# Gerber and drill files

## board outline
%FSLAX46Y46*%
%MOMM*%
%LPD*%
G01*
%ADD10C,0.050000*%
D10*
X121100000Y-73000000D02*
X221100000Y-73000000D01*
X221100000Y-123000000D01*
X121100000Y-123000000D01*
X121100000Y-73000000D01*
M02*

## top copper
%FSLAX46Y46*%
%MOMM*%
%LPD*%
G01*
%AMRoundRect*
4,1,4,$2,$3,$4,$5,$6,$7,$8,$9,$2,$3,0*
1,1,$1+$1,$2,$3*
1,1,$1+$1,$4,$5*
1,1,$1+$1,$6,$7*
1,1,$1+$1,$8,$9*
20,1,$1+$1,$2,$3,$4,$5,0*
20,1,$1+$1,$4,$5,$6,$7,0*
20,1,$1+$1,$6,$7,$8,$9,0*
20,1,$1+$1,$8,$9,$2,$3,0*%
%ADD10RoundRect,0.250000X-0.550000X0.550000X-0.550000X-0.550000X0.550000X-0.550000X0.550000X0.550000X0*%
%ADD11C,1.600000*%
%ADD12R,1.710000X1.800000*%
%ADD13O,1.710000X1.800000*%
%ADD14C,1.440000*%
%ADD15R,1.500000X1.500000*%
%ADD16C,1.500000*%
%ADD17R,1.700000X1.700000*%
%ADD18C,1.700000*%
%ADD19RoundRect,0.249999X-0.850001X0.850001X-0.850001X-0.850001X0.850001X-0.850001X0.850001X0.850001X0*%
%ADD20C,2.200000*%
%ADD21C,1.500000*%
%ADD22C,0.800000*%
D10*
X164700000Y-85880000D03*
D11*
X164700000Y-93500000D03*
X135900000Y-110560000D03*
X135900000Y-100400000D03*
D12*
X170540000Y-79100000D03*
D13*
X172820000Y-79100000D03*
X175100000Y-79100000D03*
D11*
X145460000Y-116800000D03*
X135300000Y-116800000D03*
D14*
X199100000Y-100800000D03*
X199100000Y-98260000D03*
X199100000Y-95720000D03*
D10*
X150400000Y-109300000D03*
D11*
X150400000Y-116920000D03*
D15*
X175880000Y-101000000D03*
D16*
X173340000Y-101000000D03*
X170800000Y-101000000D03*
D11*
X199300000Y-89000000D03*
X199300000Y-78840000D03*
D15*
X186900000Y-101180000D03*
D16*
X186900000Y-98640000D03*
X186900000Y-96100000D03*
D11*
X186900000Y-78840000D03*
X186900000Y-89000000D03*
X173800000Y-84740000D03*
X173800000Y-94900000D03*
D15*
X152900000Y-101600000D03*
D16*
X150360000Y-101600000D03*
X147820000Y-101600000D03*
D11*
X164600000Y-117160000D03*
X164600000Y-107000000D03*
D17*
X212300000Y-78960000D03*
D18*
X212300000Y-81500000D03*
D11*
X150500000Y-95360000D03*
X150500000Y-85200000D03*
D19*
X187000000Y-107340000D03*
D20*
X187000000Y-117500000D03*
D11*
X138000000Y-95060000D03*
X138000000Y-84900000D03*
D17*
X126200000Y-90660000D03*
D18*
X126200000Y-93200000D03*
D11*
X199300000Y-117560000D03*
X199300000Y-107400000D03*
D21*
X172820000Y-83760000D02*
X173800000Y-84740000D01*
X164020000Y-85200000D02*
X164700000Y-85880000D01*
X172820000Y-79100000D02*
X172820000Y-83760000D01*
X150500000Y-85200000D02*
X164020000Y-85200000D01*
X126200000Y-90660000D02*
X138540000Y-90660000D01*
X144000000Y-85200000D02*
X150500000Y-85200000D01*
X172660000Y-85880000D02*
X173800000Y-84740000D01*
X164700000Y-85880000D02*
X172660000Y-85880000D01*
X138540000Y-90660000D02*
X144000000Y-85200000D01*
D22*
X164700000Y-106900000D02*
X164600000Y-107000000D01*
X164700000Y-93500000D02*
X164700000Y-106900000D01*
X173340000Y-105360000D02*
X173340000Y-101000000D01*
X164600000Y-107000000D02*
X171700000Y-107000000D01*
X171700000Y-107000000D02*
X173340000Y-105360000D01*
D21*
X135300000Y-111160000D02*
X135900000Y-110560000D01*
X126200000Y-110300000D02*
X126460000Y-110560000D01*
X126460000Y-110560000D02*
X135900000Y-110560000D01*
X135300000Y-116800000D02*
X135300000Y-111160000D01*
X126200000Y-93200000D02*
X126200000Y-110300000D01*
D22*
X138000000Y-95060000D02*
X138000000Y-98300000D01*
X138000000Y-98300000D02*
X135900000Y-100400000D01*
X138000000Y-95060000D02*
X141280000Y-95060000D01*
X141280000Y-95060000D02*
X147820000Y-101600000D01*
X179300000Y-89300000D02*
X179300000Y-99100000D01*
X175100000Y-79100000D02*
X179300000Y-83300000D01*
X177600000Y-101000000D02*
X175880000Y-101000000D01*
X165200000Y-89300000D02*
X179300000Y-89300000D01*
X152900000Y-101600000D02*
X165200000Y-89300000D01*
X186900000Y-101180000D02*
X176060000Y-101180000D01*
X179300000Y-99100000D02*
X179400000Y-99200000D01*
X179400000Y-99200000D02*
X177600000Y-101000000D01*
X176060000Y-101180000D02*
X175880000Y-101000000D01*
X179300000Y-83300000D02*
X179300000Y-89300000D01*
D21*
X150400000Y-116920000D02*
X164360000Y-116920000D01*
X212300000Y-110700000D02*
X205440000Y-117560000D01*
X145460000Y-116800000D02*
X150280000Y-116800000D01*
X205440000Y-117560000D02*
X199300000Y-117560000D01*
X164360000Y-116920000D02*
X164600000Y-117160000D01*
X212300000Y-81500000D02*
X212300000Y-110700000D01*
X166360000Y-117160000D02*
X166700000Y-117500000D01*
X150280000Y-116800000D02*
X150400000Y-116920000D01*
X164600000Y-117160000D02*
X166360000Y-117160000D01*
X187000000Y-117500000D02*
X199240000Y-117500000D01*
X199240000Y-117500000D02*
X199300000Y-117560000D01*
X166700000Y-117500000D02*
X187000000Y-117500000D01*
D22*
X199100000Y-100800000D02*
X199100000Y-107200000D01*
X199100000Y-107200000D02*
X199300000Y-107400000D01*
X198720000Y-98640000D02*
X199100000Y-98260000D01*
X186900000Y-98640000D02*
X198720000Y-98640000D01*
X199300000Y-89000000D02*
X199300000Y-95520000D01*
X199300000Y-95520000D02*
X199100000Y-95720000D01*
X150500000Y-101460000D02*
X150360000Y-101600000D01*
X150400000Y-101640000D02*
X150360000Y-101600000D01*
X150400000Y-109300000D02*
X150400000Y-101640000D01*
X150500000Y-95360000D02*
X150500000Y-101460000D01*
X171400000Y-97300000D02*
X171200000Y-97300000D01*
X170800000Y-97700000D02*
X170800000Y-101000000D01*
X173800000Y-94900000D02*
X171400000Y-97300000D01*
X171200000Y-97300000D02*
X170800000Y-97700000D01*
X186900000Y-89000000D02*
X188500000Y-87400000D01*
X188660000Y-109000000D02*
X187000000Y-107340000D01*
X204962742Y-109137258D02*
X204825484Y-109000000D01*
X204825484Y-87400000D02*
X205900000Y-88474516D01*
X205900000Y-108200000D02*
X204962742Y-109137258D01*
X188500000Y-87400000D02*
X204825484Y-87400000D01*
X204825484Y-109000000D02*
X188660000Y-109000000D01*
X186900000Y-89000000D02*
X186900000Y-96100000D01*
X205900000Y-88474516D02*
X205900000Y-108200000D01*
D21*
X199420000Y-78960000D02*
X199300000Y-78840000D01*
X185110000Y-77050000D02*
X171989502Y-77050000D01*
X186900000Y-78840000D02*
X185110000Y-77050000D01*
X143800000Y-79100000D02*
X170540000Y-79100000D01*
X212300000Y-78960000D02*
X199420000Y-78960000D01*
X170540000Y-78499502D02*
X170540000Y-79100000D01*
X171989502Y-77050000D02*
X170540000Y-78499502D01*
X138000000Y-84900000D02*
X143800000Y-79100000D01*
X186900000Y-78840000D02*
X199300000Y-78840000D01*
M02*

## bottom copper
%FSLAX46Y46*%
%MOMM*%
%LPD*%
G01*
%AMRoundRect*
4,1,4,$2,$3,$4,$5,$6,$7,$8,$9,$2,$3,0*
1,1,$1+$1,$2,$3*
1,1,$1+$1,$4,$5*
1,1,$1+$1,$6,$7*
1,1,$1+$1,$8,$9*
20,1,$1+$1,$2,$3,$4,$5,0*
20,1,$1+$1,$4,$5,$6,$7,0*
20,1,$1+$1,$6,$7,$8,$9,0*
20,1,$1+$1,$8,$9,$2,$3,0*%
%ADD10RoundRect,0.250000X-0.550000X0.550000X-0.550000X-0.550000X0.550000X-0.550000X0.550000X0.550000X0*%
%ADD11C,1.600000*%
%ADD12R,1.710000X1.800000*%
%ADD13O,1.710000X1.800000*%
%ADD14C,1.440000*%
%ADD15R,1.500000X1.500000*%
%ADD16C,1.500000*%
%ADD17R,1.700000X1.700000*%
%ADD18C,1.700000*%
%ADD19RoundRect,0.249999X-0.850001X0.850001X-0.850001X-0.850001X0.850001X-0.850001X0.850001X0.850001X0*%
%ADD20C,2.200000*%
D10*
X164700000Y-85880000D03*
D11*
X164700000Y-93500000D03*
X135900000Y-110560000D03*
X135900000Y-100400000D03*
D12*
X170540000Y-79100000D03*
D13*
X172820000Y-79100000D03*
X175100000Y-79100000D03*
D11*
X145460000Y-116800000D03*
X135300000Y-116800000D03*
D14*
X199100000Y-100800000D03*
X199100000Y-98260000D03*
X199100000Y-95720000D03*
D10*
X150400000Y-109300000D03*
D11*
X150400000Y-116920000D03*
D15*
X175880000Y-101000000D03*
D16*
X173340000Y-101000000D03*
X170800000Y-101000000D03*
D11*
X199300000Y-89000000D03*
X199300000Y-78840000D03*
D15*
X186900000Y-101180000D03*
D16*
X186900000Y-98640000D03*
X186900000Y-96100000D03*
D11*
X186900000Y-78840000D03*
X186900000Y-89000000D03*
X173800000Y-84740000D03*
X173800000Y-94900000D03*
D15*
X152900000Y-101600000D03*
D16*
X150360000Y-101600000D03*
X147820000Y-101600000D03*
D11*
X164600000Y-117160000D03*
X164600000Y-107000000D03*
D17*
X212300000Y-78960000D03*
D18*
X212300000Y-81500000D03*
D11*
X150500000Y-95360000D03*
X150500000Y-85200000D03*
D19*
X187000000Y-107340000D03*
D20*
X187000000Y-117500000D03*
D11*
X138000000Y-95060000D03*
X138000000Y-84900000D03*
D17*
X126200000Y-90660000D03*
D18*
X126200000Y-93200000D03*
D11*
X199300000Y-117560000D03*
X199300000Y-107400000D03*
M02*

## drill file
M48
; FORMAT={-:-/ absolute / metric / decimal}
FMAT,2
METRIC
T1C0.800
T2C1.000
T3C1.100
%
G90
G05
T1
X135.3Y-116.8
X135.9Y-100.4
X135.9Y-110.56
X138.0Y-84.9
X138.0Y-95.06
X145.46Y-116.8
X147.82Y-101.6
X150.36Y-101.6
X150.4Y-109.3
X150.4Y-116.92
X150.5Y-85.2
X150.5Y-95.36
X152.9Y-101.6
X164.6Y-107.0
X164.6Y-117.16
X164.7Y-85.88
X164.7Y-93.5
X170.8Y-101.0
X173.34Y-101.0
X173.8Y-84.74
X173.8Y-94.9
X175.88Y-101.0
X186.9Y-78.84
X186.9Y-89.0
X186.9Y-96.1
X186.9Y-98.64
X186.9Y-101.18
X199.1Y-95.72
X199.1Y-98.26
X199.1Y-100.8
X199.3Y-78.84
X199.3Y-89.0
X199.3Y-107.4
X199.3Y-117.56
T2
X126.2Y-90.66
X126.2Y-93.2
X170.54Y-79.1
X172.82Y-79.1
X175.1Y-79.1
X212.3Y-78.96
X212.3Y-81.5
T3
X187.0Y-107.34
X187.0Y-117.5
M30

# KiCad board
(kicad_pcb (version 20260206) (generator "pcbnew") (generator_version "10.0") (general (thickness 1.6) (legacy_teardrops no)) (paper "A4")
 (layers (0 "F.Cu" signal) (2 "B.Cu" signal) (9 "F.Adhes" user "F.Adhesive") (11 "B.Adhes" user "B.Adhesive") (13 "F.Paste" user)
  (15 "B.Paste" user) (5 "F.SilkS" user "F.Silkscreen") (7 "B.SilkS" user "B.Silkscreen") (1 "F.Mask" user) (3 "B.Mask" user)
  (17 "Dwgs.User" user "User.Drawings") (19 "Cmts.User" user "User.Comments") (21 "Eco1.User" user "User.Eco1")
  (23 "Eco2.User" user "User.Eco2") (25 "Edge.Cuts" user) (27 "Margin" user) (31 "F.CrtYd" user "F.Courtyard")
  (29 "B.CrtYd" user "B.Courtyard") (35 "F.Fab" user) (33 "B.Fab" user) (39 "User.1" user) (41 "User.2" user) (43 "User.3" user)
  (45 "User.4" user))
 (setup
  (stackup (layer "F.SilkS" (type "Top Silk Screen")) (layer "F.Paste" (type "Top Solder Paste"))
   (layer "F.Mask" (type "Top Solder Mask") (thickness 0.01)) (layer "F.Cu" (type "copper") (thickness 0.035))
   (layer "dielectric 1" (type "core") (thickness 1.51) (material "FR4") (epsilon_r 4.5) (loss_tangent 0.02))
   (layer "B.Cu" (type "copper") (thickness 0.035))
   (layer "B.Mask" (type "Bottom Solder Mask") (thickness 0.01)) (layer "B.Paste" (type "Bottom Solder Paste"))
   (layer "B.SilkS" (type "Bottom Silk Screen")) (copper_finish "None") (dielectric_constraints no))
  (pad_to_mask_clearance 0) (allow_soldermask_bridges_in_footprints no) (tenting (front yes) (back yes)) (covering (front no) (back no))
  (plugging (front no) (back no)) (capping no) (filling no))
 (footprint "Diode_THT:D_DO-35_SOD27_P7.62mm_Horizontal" (layer "F.Cu") (at 164.7 85.88 -90)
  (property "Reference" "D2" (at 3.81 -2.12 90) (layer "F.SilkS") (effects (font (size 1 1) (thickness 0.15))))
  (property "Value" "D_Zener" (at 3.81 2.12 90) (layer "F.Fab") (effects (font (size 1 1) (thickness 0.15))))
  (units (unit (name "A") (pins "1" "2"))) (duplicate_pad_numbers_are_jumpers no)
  (pad "1" thru_hole roundrect (at 0 0 270) (size 1.6 1.6) (drill 0.8) (layers "*.Cu" "*.Mask") (remove_unused_layers no)
   (roundrect_rratio 0.15625) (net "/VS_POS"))
  (pad "2" thru_hole circle (at 7.62 0 270) (size 1.6 1.6) (drill 0.8) (layers "*.Cu" "*.Mask") (remove_unused_layers no) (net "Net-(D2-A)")))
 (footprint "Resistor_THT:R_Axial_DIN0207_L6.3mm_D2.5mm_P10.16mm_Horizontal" (layer "F.Cu") (at 135.9 110.56 90)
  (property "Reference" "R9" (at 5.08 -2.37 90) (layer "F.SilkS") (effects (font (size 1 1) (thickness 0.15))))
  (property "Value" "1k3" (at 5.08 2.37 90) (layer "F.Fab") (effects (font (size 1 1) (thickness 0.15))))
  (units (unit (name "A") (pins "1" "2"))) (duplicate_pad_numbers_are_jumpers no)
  (pad "1" thru_hole circle (at 0 0 90) (size 1.6 1.6) (drill 0.8) (layers "*.Cu" "*.Mask") (remove_unused_layers no) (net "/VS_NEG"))
  (pad "2" thru_hole circle (at 10.16 0 90) (size 1.6 1.6) (drill 0.8) (layers "*.Cu" "*.Mask") (remove_unused_layers no) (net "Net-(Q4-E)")))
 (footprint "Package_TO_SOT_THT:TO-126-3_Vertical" (layer "F.Cu") (at 170.54 79.1)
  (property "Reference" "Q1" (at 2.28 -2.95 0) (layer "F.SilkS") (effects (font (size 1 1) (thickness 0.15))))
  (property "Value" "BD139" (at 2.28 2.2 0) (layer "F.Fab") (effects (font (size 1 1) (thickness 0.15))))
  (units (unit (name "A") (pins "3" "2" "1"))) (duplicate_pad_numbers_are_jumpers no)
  (pad "1" thru_hole rect (at 0 0) (size 1.71 1.8) (drill 1) (layers "*.Cu" "*.Mask") (remove_unused_layers no) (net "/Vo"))
  (pad "2" thru_hole oval (at 2.28 0) (size 1.71 1.8) (drill 1) (layers "*.Cu" "*.Mask") (remove_unused_layers no) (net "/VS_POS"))
  (pad "3" thru_hole oval (at 4.56 0) (size 1.71 1.8) (drill 1) (layers "*.Cu" "*.Mask") (remove_unused_layers no) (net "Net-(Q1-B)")))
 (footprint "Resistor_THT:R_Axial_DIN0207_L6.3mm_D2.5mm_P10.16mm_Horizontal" (layer "F.Cu") (at 145.46 116.8 180)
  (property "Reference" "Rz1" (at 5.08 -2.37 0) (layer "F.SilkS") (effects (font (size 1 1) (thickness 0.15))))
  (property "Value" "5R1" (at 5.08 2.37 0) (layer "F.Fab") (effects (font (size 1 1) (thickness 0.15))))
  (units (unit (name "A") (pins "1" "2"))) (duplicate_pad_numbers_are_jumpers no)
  (pad "1" thru_hole circle (at 0 0 180) (size 1.6 1.6) (drill 0.8) (layers "*.Cu" "*.Mask") (remove_unused_layers no) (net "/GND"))
  (pad "2" thru_hole circle (at 10.16 0 180) (size 1.6 1.6) (drill 0.8) (layers "*.Cu" "*.Mask") (remove_unused_layers no) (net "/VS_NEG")))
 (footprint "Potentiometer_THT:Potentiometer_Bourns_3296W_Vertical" (layer "F.Cu") (at 199.1 100.8 -90)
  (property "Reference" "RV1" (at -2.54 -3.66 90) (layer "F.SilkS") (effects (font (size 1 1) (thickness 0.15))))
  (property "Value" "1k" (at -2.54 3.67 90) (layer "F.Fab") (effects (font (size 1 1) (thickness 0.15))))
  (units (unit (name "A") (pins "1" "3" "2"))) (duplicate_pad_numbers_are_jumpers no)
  (pad "1" thru_hole circle (at 0 0 270) (size 1.44 1.44) (drill 0.8) (layers "*.Cu" "*.Mask") (remove_unused_layers no)
   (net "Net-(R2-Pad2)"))
  (pad "2" thru_hole circle (at -2.54 0 270) (size 1.44 1.44) (drill 0.8) (layers "*.Cu" "*.Mask") (remove_unused_layers no)
   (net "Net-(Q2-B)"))
  (pad "3" thru_hole circle (at -5.08 0 270) (size 1.44 1.44) (drill 0.8) (layers "*.Cu" "*.Mask") (remove_unused_layers no)
   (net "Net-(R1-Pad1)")))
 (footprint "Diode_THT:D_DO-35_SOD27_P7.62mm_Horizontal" (layer "F.Cu") (at 150.4 109.3 -90)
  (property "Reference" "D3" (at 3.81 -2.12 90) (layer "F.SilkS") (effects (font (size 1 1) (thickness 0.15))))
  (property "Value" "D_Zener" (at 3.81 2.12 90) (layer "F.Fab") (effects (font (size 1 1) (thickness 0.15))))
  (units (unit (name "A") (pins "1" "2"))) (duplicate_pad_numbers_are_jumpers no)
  (pad "1" thru_hole roundrect (at 0 0 270) (size 1.6 1.6) (drill 0.8) (layers "*.Cu" "*.Mask") (remove_unused_layers no)
   (roundrect_rratio 0.15625) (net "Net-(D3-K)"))
  (pad "2" thru_hole circle (at 7.62 0 270) (size 1.6 1.6) (drill 0.8) (layers "*.Cu" "*.Mask") (remove_unused_layers no) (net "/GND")))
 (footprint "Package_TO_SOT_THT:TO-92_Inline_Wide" (layer "F.Cu") (at 175.88 101 180)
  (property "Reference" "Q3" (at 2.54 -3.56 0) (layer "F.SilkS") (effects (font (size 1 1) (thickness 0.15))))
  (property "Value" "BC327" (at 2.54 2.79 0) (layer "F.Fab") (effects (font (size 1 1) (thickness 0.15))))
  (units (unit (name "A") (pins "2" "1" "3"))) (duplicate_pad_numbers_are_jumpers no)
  (pad "1" thru_hole rect (at 0 0 180) (size 1.5 1.5) (drill 0.8) (layers "*.Cu" "*.Mask") (remove_unused_layers no) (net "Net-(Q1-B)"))
  (pad "2" thru_hole circle (at 2.54 0 180) (size 1.5 1.5) (drill 0.8) (layers "*.Cu" "*.Mask") (remove_unused_layers no) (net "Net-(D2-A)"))
  (pad "3" thru_hole circle (at 5.08 0 180) (size 1.5 1.5) (drill 0.8) (layers "*.Cu" "*.Mask") (remove_unused_layers no) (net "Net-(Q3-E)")))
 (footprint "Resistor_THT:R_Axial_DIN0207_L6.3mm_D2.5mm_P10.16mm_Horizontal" (layer "F.Cu") (at 199.3 89 90)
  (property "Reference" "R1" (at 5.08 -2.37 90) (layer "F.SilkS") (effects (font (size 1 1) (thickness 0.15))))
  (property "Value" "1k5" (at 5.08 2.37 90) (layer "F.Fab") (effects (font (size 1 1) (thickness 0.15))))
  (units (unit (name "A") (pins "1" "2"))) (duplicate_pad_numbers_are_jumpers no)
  (pad "1" thru_hole circle (at 0 0 90) (size 1.6 1.6) (drill 0.8) (layers "*.Cu" "*.Mask") (remove_unused_layers no) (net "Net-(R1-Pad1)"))
  (pad "2" thru_hole circle (at 10.16 0 90) (size 1.6 1.6) (drill 0.8) (layers "*.Cu" "*.Mask") (remove_unused_layers no) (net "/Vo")))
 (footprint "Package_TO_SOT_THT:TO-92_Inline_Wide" (layer "F.Cu") (at 186.9 101.18 90)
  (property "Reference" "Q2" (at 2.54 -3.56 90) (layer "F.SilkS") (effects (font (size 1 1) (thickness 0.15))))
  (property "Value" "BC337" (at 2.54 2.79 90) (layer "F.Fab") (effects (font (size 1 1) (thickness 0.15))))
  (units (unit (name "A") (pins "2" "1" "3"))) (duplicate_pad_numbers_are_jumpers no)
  (pad "1" thru_hole rect (at 0 0 90) (size 1.5 1.5) (drill 0.8) (layers "*.Cu" "*.Mask") (remove_unused_layers no) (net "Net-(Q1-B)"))
  (pad "2" thru_hole circle (at 2.54 0 90) (size 1.5 1.5) (drill 0.8) (layers "*.Cu" "*.Mask") (remove_unused_layers no) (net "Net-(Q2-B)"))
  (pad "3" thru_hole circle (at 5.08 0 90) (size 1.5 1.5) (drill 0.8) (layers "*.Cu" "*.Mask") (remove_unused_layers no) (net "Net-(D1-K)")))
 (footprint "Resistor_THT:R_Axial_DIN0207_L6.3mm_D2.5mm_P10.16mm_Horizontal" (layer "F.Cu") (at 186.9 78.84 -90)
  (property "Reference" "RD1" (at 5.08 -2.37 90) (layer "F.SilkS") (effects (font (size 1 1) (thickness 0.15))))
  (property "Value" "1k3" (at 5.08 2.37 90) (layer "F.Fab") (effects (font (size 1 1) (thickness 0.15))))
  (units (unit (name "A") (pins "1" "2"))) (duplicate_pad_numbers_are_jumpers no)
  (pad "1" thru_hole circle (at 0 0 270) (size 1.6 1.6) (drill 0.8) (layers "*.Cu" "*.Mask") (remove_unused_layers no) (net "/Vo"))
  (pad "2" thru_hole circle (at 10.16 0 270) (size 1.6 1.6) (drill 0.8) (layers "*.Cu" "*.Mask") (remove_unused_layers no)
   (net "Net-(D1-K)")))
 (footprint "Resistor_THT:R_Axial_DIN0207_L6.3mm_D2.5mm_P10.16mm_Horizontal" (layer "F.Cu") (at 173.8 84.74 -90)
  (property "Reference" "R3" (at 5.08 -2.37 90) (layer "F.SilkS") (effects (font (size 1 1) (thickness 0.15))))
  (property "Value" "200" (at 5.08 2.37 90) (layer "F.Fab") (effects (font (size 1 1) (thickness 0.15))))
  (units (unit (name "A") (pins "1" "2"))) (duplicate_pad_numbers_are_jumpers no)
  (pad "1" thru_hole circle (at 0 0 270) (size 1.6 1.6) (drill 0.8) (layers "*.Cu" "*.Mask") (remove_unused_layers no) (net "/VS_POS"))
  (pad "2" thru_hole circle (at 10.16 0 270) (size 1.6 1.6) (drill 0.8) (layers "*.Cu" "*.Mask") (remove_unused_layers no)
   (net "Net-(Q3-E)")))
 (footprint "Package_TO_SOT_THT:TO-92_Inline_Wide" (layer "F.Cu") (at 152.9 101.6 180)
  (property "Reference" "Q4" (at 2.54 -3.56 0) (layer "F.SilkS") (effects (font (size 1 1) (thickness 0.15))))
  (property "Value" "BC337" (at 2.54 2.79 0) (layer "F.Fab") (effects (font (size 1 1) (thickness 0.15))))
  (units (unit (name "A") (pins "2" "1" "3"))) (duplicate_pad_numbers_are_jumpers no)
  (pad "1" thru_hole rect (at 0 0 180) (size 1.5 1.5) (drill 0.8) (layers "*.Cu" "*.Mask") (remove_unused_layers no) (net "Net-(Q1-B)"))
  (pad "2" thru_hole circle (at 2.54 0 180) (size 1.5 1.5) (drill 0.8) (layers "*.Cu" "*.Mask") (remove_unused_layers no) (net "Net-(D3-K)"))
  (pad "3" thru_hole circle (at 5.08 0 180) (size 1.5 1.5) (drill 0.8) (layers "*.Cu" "*.Mask") (remove_unused_layers no) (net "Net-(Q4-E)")))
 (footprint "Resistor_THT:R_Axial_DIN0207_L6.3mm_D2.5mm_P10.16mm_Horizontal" (layer "F.Cu") (at 164.6 117.16 90)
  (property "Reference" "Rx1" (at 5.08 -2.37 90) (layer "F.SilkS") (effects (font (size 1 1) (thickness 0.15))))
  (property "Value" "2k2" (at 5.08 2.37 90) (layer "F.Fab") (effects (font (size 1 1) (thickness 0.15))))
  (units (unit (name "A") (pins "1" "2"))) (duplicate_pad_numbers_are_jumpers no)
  (pad "1" thru_hole circle (at 0 0 90) (size 1.6 1.6) (drill 0.8) (layers "*.Cu" "*.Mask") (remove_unused_layers no) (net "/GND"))
  (pad "2" thru_hole circle (at 10.16 0 90) (size 1.6 1.6) (drill 0.8) (layers "*.Cu" "*.Mask") (remove_unused_layers no) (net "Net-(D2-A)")))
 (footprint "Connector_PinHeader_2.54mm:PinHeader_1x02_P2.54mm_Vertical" (layer "F.Cu") (at 212.3 78.96)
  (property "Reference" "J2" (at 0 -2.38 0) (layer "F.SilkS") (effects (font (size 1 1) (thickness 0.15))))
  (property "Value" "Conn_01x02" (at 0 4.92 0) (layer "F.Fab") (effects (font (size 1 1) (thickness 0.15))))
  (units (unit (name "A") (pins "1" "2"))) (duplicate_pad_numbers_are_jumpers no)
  (pad "1" thru_hole rect (at 0 0) (size 1.7 1.7) (drill 1) (layers "*.Cu" "*.Mask") (remove_unused_layers no) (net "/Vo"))
  (pad "2" thru_hole circle (at 0 2.54) (size 1.7 1.7) (drill 1) (layers "*.Cu" "*.Mask") (remove_unused_layers no) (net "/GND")))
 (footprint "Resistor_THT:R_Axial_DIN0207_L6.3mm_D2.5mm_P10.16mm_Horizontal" (layer "F.Cu") (at 150.5 95.36 90)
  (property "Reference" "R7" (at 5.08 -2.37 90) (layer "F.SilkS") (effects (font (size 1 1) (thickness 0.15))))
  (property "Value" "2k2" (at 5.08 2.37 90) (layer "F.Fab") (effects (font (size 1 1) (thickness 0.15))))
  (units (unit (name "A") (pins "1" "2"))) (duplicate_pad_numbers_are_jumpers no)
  (pad "1" thru_hole circle (at 0 0 90) (size 1.6 1.6) (drill 0.8) (layers "*.Cu" "*.Mask") (remove_unused_layers no) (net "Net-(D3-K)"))
  (pad "2" thru_hole circle (at 10.16 0 90) (size 1.6 1.6) (drill 0.8) (layers "*.Cu" "*.Mask") (remove_unused_layers no) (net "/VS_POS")))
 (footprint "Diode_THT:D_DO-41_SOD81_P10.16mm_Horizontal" (layer "F.Cu") (at 187 107.34 -90)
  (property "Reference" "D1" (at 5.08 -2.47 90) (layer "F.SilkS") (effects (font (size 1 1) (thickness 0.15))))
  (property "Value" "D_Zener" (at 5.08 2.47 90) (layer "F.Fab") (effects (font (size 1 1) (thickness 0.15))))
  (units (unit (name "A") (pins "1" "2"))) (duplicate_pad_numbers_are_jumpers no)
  (pad "1" thru_hole roundrect (at 0 0 270) (size 2.2 2.2) (drill 1.1) (layers "*.Cu" "*.Mask") (remove_unused_layers no)
   (roundrect_rratio 0.113636) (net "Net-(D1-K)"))
  (pad "2" thru_hole circle (at 10.16 0 270) (size 2.2 2.2) (drill 1.1) (layers "*.Cu" "*.Mask") (remove_unused_layers no) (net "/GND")))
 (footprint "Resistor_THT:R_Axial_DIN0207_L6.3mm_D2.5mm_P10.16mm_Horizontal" (layer "F.Cu") (at 138 95.06 90)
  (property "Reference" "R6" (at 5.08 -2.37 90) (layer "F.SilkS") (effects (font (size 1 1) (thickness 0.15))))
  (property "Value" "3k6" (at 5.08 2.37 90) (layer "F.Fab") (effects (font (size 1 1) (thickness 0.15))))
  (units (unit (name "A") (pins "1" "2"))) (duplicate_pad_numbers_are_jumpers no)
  (pad "1" thru_hole circle (at 0 0 90) (size 1.6 1.6) (drill 0.8) (layers "*.Cu" "*.Mask") (remove_unused_layers no) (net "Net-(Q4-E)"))
  (pad "2" thru_hole circle (at 10.16 0 90) (size 1.6 1.6) (drill 0.8) (layers "*.Cu" "*.Mask") (remove_unused_layers no) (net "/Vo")))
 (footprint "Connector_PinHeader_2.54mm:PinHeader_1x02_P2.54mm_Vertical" (layer "F.Cu") (at 126.2 90.66)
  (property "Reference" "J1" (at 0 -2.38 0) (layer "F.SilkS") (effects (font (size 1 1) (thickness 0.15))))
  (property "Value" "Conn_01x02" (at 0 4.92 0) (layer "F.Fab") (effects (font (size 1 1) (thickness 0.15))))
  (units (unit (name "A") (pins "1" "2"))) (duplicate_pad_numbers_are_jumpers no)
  (pad "1" thru_hole rect (at 0 0) (size 1.7 1.7) (drill 1) (layers "*.Cu" "*.Mask") (remove_unused_layers no) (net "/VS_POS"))
  (pad "2" thru_hole circle (at 0 2.54) (size 1.7 1.7) (drill 1) (layers "*.Cu" "*.Mask") (remove_unused_layers no) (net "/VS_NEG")))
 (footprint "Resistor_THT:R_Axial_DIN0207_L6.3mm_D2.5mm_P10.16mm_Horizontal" (layer "F.Cu") (at 199.3 117.56 90)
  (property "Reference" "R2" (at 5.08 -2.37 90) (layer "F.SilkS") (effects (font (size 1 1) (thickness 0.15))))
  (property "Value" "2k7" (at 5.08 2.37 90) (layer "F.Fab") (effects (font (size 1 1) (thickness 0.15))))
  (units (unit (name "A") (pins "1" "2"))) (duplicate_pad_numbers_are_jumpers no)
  (pad "1" thru_hole circle (at 0 0 90) (size 1.6 1.6) (drill 0.8) (layers "*.Cu" "*.Mask") (remove_unused_layers no) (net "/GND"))
  (pad "2" thru_hole circle (at 10.16 0 90) (size 1.6 1.6) (drill 0.8) (layers "*.Cu" "*.Mask") (remove_unused_layers no)
   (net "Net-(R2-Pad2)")))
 (gr_rect (start 121.1 73) (end 221.1 123) (stroke (width 0.05) (type default)) (fill no) (layer "Edge.Cuts"))
 (segment (start 172.82 83.76) (end 173.8 84.74) (width 1.5) (layer "F.Cu") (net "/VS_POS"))
 (segment (start 164.02 85.2) (end 164.7 85.88) (width 1.5) (layer "F.Cu") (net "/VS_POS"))
 (segment (start 172.82 79.1) (end 172.82 83.76) (width 1.5) (layer "F.Cu") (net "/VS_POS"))
 (segment (start 150.5 85.2) (end 164.02 85.2) (width 1.5) (layer "F.Cu") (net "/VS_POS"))
 (segment (start 126.2 90.66) (end 138.54 90.66) (width 1.5) (layer "F.Cu") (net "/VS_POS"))
 (segment (start 144 85.2) (end 150.5 85.2) (width 1.5) (layer "F.Cu") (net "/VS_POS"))
 (segment (start 172.66 85.88) (end 173.8 84.74) (width 1.5) (layer "F.Cu") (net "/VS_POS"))
 (segment (start 164.7 85.88) (end 172.66 85.88) (width 1.5) (layer "F.Cu") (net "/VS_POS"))
 (segment (start 138.54 90.66) (end 144 85.2) (width 1.5) (layer "F.Cu") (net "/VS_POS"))
 (segment (start 164.7 106.9) (end 164.6 107) (width 0.8) (layer "F.Cu") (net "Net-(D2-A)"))
 (segment (start 164.7 93.5) (end 164.7 106.9) (width 0.8) (layer "F.Cu") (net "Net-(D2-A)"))
 (segment (start 173.34 105.36) (end 173.34 101) (width 0.8) (layer "F.Cu") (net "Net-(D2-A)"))
 (segment (start 164.6 107) (end 171.7 107) (width 0.8) (layer "F.Cu") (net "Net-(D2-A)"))
 (segment (start 171.7 107) (end 173.34 105.36) (width 0.8) (layer "F.Cu") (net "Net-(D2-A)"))
 (segment (start 135.3 111.16) (end 135.9 110.56) (width 1.5) (layer "F.Cu") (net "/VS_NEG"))
 (segment (start 126.2 110.3) (end 126.46 110.56) (width 1.5) (layer "F.Cu") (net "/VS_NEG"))
 (segment (start 126.46 110.56) (end 135.9 110.56) (width 1.5) (layer "F.Cu") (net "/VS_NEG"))
 (segment (start 135.3 116.8) (end 135.3 111.16) (width 1.5) (layer "F.Cu") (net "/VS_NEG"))
 (segment (start 126.2 93.2) (end 126.2 110.3) (width 1.5) (layer "F.Cu") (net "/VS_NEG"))
 (segment (start 138 95.06) (end 138 98.3) (width 0.8) (layer "F.Cu") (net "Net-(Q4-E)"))
 (segment (start 138 98.3) (end 135.9 100.4) (width 0.8) (layer "F.Cu") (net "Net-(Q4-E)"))
 (segment (start 138 95.06) (end 141.28 95.06) (width 0.8) (layer "F.Cu") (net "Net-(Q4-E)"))
 (segment (start 141.28 95.06) (end 147.82 101.6) (width 0.8) (layer "F.Cu") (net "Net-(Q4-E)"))
 (segment (start 179.3 89.3) (end 179.3 99.1) (width 0.8) (layer "F.Cu") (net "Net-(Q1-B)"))
 (segment (start 175.1 79.1) (end 179.3 83.3) (width 0.8) (layer "F.Cu") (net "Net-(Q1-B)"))
 (segment (start 177.6 101) (end 175.88 101) (width 0.8) (layer "F.Cu") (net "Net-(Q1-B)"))
 (segment (start 165.2 89.3) (end 179.3 89.3) (width 0.8) (layer "F.Cu") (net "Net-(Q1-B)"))
 (segment (start 152.9 101.6) (end 165.2 89.3) (width 0.8) (layer "F.Cu") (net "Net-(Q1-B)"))
 (segment (start 186.9 101.18) (end 176.06 101.18) (width 0.8) (layer "F.Cu") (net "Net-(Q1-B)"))
 (segment (start 179.3 99.1) (end 179.4 99.2) (width 0.8) (layer "F.Cu") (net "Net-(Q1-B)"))
 (segment (start 179.4 99.2) (end 177.6 101) (width 0.8) (layer "F.Cu") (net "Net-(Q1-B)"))
 (segment (start 176.06 101.18) (end 175.88 101) (width 0.8) (layer "F.Cu") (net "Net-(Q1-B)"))
 (segment (start 179.3 83.3) (end 179.3 89.3) (width 0.8) (layer "F.Cu") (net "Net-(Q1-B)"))
 (segment (start 150.4 116.92) (end 164.36 116.92) (width 1.5) (layer "F.Cu") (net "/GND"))
 (segment (start 212.3 110.7) (end 205.44 117.56) (width 1.5) (layer "F.Cu") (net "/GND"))
 (segment (start 145.46 116.8) (end 150.28 116.8) (width 1.5) (layer "F.Cu") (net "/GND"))
 (segment (start 205.44 117.56) (end 199.3 117.56) (width 1.5) (layer "F.Cu") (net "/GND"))
 (segment (start 164.36 116.92) (end 164.6 117.16) (width 1.5) (layer "F.Cu") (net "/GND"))
 (segment (start 212.3 81.5) (end 212.3 110.7) (width 1.5) (layer "F.Cu") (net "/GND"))
 (segment (start 166.36 117.16) (end 166.7 117.5) (width 1.5) (layer "F.Cu") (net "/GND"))
 (segment (start 150.28 116.8) (end 150.4 116.92) (width 1.5) (layer "F.Cu") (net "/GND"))
 (segment (start 164.6 117.16) (end 166.36 117.16) (width 1.5) (layer "F.Cu") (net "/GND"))
 (segment (start 187 117.5) (end 199.24 117.5) (width 1.5) (layer "F.Cu") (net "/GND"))
 (segment (start 199.24 117.5) (end 199.3 117.56) (width 1.5) (layer "F.Cu") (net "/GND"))
 (segment (start 166.7 117.5) (end 187 117.5) (width 1.5) (layer "F.Cu") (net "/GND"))
 (segment (start 199.1 100.8) (end 199.1 107.2) (width 0.8) (layer "F.Cu") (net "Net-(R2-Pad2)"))
 (segment (start 199.1 107.2) (end 199.3 107.4) (width 0.8) (layer "F.Cu") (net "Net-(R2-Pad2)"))
 (segment (start 198.72 98.64) (end 199.1 98.26) (width 0.8) (layer "F.Cu") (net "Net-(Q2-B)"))
 (segment (start 186.9 98.64) (end 198.72 98.64) (width 0.8) (layer "F.Cu") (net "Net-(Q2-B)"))
 (segment (start 199.3 89) (end 199.3 95.52) (width 0.8) (layer "F.Cu") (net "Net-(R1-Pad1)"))
 (segment (start 199.3 95.52) (end 199.1 95.72) (width 0.8) (layer "F.Cu") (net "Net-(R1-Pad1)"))
 (segment (start 150.5 101.46) (end 150.36 101.6) (width 0.8) (layer "F.Cu") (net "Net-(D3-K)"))
 (segment (start 150.4 101.64) (end 150.36 101.6) (width 0.8) (layer "F.Cu") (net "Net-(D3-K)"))
 (segment (start 150.4 109.3) (end 150.4 101.64) (width 0.8) (layer "F.Cu") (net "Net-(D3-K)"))
 (segment (start 150.5 95.36) (end 150.5 101.46) (width 0.8) (layer "F.Cu") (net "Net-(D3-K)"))
 (segment (start 171.4 97.3) (end 171.2 97.3) (width 0.8) (layer "F.Cu") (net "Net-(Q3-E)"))
 (segment (start 170.8 97.7) (end 170.8 101) (width 0.8) (layer "F.Cu") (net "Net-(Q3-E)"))
 (segment (start 173.8 94.9) (end 171.4 97.3) (width 0.8) (layer "F.Cu") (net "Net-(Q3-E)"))
 (segment (start 171.2 97.3) (end 170.8 97.7) (width 0.8) (layer "F.Cu") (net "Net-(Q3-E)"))
 (segment (start 186.9 89) (end 188.5 87.4) (width 0.8) (layer "F.Cu") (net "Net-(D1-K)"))
 (segment (start 188.66 109) (end 187 107.34) (width 0.8) (layer "F.Cu") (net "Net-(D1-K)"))
 (segment (start 204.962742 109.137258) (end 204.825484 109) (width 0.8) (layer "F.Cu") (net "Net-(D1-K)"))
 (segment (start 204.825484 87.4) (end 205.9 88.474516) (width 0.8) (layer "F.Cu") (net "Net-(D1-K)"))
 (segment (start 205.9 108.2) (end 204.962742 109.137258) (width 0.8) (layer "F.Cu") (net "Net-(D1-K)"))
 (segment (start 188.5 87.4) (end 204.825484 87.4) (width 0.8) (layer "F.Cu") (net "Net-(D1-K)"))
 (segment (start 204.825484 109) (end 188.66 109) (width 0.8) (layer "F.Cu") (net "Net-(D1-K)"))
 (segment (start 186.9 89) (end 186.9 96.1) (width 0.8) (layer "F.Cu") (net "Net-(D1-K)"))
 (segment (start 205.9 88.474516) (end 205.9 108.2) (width 0.8) (layer "F.Cu") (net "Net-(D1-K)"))
 (segment (start 199.42 78.96) (end 199.3 78.84) (width 1.5) (layer "F.Cu") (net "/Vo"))
 (segment (start 185.11 77.05) (end 171.989502 77.05) (width 1.5) (layer "F.Cu") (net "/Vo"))
 (segment (start 186.9 78.84) (end 185.11 77.05) (width 1.5) (layer "F.Cu") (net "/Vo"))
 (segment (start 143.8 79.1) (end 170.54 79.1) (width 1.5) (layer "F.Cu") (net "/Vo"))
 (segment (start 212.3 78.96) (end 199.42 78.96) (width 1.5) (layer "F.Cu") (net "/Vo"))
 (segment (start 170.54 78.499502) (end 170.54 79.1) (width 1.5) (layer "F.Cu") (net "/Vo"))
 (segment (start 171.989502 77.05) (end 170.54 78.499502) (width 1.5) (layer "F.Cu") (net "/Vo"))
 (segment (start 138 84.9) (end 143.8 79.1) (width 1.5) (layer "F.Cu") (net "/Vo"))
 (segment (start 186.9 78.84) (end 199.3 78.84) (width 1.5) (layer "F.Cu") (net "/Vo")))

